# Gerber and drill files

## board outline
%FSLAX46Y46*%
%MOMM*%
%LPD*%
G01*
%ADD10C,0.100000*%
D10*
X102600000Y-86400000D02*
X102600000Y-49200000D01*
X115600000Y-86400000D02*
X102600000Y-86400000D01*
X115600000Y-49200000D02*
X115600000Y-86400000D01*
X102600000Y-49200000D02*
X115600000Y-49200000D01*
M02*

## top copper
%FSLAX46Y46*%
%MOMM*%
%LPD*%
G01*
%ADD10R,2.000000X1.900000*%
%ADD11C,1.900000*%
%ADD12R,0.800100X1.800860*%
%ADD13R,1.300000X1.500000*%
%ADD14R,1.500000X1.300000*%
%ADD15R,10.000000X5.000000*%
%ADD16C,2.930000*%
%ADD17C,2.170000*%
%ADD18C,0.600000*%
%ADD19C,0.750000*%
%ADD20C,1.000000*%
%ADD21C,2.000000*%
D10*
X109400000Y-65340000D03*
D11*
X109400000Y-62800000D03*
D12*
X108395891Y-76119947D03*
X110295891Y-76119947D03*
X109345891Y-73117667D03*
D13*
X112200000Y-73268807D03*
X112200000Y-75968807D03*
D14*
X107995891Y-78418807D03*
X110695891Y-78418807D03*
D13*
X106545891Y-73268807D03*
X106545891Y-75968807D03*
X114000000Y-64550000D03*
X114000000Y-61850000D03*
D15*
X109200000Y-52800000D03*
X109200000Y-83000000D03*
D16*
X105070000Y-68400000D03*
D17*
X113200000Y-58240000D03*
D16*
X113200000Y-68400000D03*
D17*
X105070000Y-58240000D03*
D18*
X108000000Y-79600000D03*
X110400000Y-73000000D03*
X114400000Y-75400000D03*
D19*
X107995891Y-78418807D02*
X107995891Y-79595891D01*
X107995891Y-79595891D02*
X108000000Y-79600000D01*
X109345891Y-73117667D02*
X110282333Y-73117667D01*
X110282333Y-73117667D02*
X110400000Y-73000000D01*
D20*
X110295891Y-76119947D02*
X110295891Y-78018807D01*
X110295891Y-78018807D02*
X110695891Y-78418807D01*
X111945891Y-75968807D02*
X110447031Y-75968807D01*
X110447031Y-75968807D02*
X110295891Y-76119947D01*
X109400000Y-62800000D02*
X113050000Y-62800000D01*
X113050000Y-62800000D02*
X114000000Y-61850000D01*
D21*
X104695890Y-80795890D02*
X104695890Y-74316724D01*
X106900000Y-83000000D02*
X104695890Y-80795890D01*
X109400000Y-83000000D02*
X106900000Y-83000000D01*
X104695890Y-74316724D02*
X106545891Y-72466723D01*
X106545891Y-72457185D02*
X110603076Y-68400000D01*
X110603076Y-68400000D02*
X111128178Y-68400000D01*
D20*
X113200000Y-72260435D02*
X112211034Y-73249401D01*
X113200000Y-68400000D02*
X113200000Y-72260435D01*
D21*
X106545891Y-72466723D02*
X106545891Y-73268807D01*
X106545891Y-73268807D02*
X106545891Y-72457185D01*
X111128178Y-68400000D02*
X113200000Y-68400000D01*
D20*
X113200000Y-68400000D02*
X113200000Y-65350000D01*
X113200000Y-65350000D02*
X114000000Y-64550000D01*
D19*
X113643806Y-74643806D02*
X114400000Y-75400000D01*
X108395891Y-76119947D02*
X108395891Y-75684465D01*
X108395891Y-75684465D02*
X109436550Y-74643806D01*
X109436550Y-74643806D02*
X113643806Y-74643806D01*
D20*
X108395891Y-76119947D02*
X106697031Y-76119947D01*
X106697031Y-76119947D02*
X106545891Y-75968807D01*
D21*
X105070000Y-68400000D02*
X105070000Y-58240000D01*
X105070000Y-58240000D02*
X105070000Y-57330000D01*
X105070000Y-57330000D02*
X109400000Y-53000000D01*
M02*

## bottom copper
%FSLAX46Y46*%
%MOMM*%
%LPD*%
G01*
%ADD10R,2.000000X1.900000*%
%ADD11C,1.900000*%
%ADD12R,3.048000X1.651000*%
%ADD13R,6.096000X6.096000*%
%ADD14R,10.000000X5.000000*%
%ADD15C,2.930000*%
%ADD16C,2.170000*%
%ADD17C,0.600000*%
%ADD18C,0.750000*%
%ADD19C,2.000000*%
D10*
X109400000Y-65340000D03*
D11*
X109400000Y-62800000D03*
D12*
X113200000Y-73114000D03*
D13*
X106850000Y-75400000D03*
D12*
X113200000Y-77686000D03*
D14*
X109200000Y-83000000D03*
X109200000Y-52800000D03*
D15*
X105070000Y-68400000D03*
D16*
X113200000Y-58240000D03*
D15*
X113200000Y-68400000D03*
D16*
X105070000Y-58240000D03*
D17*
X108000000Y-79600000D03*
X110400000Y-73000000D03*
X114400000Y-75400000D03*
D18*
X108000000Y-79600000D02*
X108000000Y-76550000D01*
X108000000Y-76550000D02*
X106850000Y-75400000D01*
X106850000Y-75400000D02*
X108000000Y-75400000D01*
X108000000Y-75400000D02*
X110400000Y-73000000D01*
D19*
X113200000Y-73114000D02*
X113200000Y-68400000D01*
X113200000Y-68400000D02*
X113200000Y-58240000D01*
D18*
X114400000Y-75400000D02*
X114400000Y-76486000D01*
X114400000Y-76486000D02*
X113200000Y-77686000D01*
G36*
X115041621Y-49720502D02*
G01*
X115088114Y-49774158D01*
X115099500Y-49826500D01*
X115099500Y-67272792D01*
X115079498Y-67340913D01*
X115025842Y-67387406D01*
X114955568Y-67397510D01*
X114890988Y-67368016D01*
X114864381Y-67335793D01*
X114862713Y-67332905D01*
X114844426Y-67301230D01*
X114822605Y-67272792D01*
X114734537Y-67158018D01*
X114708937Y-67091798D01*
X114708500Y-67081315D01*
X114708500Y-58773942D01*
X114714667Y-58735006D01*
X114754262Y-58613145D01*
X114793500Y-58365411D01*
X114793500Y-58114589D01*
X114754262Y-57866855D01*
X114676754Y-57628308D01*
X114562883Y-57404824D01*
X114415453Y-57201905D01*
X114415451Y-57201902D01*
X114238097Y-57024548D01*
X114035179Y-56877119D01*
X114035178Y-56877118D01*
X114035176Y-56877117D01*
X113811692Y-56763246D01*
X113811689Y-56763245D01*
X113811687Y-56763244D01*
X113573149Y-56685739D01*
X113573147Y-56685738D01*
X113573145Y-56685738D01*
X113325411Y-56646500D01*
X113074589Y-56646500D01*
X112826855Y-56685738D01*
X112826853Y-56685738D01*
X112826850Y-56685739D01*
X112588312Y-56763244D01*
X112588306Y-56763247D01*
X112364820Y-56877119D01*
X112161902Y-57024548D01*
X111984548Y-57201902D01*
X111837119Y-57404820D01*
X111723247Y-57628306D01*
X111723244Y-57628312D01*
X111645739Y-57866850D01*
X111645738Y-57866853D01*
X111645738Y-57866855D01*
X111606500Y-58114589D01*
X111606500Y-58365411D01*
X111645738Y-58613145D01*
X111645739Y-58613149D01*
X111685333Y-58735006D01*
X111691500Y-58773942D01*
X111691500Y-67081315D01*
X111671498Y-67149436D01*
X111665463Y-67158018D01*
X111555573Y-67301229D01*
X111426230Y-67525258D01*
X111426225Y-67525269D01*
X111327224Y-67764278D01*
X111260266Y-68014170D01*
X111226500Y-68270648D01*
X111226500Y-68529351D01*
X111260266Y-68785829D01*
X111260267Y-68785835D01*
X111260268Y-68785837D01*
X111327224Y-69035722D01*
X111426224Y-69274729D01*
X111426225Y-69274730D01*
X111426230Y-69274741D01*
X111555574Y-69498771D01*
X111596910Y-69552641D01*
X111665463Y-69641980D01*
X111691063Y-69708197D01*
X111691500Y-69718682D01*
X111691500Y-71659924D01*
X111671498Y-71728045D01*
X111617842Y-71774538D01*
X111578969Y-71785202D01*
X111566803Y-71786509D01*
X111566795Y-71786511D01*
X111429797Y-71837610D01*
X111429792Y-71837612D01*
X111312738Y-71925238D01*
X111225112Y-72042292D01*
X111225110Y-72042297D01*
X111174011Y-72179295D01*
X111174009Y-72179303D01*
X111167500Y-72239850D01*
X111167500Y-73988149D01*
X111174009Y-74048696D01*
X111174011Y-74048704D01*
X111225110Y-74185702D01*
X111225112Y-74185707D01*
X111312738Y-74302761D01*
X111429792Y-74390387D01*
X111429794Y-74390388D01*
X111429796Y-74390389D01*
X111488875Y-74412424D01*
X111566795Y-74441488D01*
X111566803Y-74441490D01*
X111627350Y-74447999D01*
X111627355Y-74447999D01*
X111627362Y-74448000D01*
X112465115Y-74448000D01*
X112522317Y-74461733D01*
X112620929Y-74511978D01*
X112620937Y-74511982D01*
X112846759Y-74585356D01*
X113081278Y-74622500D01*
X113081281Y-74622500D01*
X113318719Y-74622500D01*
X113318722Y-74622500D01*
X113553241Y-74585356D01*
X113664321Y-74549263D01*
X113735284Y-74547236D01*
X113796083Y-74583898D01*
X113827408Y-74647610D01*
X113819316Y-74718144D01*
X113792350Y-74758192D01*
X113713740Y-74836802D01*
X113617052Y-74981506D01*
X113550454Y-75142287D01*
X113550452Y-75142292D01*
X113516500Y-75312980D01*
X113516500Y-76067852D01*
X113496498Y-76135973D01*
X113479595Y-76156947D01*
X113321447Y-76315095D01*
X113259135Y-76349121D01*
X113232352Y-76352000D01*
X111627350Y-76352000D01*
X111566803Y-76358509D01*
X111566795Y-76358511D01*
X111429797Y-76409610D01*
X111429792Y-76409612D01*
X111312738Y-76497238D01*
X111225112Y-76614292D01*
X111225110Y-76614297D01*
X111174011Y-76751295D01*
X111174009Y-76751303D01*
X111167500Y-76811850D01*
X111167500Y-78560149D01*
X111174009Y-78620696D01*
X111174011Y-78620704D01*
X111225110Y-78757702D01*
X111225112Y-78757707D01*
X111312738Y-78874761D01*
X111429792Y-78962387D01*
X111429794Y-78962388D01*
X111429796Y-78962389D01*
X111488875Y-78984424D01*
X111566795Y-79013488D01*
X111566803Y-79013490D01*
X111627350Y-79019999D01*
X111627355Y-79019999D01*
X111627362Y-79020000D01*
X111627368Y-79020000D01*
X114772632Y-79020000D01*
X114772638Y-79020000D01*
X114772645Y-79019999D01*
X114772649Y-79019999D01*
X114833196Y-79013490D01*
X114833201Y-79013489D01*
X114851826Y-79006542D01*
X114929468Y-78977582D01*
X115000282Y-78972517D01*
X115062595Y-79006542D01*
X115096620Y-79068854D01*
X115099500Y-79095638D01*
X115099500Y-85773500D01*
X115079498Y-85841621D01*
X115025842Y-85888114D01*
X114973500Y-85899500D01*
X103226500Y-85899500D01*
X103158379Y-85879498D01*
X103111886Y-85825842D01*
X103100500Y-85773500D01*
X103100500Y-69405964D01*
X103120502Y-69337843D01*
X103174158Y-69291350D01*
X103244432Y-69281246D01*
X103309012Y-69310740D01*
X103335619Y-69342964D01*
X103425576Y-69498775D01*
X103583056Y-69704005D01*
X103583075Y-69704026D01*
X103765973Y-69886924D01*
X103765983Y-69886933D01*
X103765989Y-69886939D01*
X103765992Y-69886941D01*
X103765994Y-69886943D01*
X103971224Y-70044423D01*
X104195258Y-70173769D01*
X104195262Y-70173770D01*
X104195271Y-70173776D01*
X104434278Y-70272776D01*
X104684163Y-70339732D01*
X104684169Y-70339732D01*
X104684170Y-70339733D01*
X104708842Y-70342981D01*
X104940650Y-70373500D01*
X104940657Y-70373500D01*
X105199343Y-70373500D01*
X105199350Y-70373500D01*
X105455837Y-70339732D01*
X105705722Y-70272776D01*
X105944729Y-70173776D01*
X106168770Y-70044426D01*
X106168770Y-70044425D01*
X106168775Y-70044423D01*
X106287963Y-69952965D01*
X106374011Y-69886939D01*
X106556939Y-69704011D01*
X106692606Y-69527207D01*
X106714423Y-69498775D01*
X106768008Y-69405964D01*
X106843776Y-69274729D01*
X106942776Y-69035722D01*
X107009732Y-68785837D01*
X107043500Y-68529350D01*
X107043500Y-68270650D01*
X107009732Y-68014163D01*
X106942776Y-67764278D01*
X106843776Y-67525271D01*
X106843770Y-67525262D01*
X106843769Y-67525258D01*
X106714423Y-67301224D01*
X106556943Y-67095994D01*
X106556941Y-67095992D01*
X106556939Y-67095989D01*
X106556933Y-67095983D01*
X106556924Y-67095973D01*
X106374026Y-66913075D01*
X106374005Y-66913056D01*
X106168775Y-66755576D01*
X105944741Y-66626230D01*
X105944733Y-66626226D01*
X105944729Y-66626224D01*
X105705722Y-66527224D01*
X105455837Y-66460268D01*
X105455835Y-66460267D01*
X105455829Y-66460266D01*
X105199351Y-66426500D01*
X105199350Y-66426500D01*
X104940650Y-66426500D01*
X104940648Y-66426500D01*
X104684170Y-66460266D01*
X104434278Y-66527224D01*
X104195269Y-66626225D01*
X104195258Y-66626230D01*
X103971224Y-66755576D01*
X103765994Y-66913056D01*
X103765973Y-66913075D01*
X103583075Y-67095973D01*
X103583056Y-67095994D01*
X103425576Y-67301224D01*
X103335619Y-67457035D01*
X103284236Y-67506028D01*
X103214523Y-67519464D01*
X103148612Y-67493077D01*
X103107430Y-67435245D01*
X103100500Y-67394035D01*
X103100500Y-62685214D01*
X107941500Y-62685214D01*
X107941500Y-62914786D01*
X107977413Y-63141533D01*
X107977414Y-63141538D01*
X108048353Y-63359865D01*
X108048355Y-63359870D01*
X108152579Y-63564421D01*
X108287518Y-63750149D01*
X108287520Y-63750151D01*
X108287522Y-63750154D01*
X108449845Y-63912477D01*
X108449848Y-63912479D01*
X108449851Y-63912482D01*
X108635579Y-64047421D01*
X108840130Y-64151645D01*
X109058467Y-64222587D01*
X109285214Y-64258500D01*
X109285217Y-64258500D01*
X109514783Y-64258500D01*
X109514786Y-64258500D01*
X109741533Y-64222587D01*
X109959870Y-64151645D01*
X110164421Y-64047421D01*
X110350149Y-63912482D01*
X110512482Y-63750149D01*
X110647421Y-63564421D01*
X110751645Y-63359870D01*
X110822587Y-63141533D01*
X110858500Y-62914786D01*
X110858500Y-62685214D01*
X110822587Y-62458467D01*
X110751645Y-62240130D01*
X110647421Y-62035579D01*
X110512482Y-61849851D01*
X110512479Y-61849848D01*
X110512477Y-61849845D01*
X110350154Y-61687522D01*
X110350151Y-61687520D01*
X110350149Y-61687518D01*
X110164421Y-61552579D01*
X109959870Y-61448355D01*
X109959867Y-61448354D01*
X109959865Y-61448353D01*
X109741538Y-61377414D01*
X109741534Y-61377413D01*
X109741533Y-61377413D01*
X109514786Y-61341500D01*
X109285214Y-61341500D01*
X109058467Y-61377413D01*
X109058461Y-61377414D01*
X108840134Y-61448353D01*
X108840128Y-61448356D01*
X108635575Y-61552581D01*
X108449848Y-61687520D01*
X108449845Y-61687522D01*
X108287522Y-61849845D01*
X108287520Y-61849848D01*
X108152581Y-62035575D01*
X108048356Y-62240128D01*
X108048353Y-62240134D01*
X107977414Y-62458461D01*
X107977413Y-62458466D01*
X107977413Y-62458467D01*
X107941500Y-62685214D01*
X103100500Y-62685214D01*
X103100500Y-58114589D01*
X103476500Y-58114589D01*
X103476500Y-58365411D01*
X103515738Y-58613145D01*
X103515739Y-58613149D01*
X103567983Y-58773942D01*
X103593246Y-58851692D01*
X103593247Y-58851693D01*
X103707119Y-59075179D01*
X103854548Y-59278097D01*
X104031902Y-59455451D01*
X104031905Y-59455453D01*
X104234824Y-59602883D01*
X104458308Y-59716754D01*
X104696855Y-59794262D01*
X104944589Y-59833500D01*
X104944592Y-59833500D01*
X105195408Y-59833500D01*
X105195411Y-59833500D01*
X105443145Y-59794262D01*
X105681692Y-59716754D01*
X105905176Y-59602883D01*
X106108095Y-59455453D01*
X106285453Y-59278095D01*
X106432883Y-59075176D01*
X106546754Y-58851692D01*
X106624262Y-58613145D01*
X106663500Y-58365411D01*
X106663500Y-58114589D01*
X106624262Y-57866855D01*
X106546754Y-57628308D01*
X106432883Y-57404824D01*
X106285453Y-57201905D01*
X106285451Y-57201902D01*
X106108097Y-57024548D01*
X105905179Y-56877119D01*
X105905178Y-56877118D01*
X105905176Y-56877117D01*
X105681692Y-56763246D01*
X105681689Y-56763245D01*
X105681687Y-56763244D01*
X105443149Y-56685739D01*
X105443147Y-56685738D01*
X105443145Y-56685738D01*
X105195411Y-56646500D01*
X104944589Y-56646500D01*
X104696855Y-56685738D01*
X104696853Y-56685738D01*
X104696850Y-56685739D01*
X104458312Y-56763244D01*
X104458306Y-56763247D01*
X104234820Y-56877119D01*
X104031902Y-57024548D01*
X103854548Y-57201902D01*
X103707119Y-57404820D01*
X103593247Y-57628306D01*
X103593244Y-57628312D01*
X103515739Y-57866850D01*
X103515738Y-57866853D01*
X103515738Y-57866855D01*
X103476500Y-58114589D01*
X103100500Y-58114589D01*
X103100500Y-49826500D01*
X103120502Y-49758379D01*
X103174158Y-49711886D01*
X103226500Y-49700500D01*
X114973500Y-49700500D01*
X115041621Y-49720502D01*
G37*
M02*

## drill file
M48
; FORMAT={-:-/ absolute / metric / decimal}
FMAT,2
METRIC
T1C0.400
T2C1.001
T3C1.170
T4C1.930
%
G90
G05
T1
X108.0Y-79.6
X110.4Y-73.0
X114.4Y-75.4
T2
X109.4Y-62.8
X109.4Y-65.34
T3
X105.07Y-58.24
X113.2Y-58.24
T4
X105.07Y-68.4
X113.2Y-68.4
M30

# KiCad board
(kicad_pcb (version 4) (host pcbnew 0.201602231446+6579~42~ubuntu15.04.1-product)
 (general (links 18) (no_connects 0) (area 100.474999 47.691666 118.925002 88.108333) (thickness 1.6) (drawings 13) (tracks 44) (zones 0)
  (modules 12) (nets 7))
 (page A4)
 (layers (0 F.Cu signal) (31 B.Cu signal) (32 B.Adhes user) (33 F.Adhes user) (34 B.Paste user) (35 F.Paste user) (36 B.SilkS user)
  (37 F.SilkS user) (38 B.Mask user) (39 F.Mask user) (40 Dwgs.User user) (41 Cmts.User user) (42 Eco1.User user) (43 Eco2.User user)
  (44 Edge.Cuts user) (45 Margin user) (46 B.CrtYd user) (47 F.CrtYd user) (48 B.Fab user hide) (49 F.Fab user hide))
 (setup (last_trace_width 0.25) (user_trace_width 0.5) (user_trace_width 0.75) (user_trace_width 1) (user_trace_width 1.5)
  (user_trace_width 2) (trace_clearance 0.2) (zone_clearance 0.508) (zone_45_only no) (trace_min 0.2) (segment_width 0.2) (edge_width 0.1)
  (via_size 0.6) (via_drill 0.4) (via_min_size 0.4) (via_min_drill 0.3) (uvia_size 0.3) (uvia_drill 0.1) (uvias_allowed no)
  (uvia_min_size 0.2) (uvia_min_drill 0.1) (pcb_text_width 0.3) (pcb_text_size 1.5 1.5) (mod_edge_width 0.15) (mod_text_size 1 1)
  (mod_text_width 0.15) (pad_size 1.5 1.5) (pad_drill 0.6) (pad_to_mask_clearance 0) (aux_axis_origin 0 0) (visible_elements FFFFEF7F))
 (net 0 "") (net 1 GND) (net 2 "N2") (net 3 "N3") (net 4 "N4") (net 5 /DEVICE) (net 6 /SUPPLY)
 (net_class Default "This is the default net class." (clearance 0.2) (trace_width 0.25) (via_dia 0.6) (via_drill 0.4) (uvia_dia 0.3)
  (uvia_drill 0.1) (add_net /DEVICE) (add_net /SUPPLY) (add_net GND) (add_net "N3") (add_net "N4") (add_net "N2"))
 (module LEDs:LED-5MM (layer F.Cu) (at 109.4 65.34 90)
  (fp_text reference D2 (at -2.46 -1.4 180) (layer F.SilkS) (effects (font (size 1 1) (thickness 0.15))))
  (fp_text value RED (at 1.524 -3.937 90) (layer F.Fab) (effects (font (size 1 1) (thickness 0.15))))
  (pad 1 thru_hole rect (at 0 0 180) (size 2 1.9) (drill 1.00076) (layers *.Cu *.Mask F.SilkS) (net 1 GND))
  (pad 2 thru_hole circle (at 2.54 0 90) (size 1.9 1.9) (drill 1.00076) (layers *.Cu *.Mask F.SilkS) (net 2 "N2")))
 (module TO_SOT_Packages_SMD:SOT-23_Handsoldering (layer F.Cu) (at 109.345891 74.618807)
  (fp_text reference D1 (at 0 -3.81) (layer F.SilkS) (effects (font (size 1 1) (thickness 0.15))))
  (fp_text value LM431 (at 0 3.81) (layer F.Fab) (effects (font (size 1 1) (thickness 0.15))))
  (pad 1 smd rect (at -0.95 1.50114) (size 0.8001 1.80086) (layers F.Cu F.Paste F.Mask) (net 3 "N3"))
  (pad 2 smd rect (at 0.95 1.50114) (size 0.8001 1.80086) (layers F.Cu F.Paste F.Mask) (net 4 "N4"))
  (pad 3 smd rect (at 0 -1.50114) (size 0.8001 1.80086) (layers F.Cu F.Paste F.Mask) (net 1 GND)))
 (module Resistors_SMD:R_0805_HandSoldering (layer F.Cu) (at 112.2 74.618807 270)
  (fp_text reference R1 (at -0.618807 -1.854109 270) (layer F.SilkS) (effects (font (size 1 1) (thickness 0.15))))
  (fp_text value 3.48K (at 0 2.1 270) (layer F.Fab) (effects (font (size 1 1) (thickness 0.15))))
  (pad 1 smd rect (at -1.35 0 270) (size 1.5 1.3) (layers F.Cu F.Paste F.Mask) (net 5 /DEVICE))
  (pad 2 smd rect (at 1.35 0 270) (size 1.5 1.3) (layers F.Cu F.Paste F.Mask) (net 4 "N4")))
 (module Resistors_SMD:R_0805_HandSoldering (layer F.Cu) (at 109.345891 78.418807)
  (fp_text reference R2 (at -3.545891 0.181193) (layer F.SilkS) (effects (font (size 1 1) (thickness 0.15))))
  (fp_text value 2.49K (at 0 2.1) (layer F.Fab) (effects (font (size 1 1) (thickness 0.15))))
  (pad 1 smd rect (at -1.35 0) (size 1.5 1.3) (layers F.Cu F.Paste F.Mask) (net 1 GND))
  (pad 2 smd rect (at 1.35 0) (size 1.5 1.3) (layers F.Cu F.Paste F.Mask) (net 4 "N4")))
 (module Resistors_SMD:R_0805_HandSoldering (layer F.Cu) (at 106.545891 74.618807 270)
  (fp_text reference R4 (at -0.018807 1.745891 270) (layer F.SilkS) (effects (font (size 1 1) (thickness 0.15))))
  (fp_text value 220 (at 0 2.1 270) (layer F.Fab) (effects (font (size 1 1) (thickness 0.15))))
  (pad 1 smd rect (at -1.35 0 270) (size 1.5 1.3) (layers F.Cu F.Paste F.Mask) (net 5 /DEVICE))
  (pad 2 smd rect (at 1.35 0 270) (size 1.5 1.3) (layers F.Cu F.Paste F.Mask) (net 3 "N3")))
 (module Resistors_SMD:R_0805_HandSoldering (layer F.Cu) (at 114 63.2 90)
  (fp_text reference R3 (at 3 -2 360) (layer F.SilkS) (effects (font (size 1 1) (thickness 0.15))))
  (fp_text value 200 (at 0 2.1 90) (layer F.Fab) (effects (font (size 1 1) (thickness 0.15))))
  (pad 1 smd rect (at -1.35 0 90) (size 1.5 1.3) (layers F.Cu F.Paste F.Mask) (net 5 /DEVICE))
  (pad 2 smd rect (at 1.35 0 90) (size 1.5 1.3) (layers F.Cu F.Paste F.Mask) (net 2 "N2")))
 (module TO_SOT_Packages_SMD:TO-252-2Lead (layer B.Cu) (at 113.2 75.4 270)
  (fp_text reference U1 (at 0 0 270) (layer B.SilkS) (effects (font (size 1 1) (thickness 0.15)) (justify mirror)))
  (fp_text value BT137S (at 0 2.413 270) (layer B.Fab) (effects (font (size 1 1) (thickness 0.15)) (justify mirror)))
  (pad 1 smd rect (at -2.286 0 270) (size 1.651 3.048) (layers B.Cu B.Paste B.Mask) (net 5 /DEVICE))
  (pad 2 smd rect (at 0 6.35 270) (size 6.096 6.096) (layers B.Cu B.Paste B.Mask) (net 1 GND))
  (pad 3 smd rect (at 2.286 0 270) (size 1.651 3.048) (layers B.Cu B.Paste B.Mask) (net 3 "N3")))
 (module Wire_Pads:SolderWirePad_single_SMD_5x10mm (layer F.Cu) (at 109.2 52.8 90)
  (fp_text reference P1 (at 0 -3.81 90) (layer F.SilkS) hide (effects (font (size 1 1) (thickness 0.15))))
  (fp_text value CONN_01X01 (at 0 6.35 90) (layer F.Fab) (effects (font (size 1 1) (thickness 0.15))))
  (pad 1 smd rect (at 0 0 90) (size 5 10) (layers F.Cu F.Paste F.Mask) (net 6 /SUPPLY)))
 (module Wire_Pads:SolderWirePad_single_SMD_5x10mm (layer F.Cu) (at 109.2 83 90)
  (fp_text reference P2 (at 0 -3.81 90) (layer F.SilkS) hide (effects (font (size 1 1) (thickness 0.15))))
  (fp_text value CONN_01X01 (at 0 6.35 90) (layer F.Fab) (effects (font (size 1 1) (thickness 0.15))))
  (pad 1 smd rect (at 0 0 90) (size 5 10) (layers F.Cu F.Paste F.Mask) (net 5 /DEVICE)))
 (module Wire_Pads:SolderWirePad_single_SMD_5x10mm (layer B.Cu) (at 109.2 83 90)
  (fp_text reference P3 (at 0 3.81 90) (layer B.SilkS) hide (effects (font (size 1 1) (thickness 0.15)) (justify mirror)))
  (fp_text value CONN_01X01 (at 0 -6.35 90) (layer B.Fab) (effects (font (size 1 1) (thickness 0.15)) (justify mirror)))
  (pad 1 smd rect (at 0 0 90) (size 5 10) (layers B.Cu B.Paste B.Mask) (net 1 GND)))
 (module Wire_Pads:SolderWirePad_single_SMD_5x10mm (layer B.Cu) (at 109.2 52.8 90)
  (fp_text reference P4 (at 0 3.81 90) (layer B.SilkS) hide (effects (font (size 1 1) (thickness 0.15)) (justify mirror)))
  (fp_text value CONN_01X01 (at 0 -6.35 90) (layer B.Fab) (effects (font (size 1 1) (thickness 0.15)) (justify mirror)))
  (pad 1 smd rect (at 0 0 90) (size 5 10) (layers B.Cu B.Paste B.Mask) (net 1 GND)))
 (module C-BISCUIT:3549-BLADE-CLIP (layer B.Cu) (at 109.135 63.32)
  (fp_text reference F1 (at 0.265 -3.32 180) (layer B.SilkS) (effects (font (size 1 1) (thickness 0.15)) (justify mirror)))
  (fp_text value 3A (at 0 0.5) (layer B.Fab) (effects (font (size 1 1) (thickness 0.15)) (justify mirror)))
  (pad 1 thru_hole circle (at -4.065 5.08) (size 2.93 2.93) (drill 1.93) (layers *.Cu *.Mask B.SilkS) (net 6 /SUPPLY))
  (pad 2 thru_hole circle (at 4.065 -5.08) (size 2.17 2.17) (drill 1.17) (layers *.Cu *.Mask B.SilkS) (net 5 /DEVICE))
  (pad 2 thru_hole circle (at 4.065 5.08) (size 2.93 2.93) (drill 1.93) (layers *.Cu *.Mask B.SilkS) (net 5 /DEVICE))
  (pad 1 thru_hole circle (at -4.065 -5.08) (size 2.17 2.17) (drill 1.17) (layers *.Cu *.Mask B.SilkS) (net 6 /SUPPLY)))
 (gr_line (start 102.6 86.4) (end 102.6 49.2) (layer Edge.Cuts) (width 0.1))
 (gr_line (start 115.6 86.4) (end 102.6 86.4) (layer Edge.Cuts) (width 0.1))
 (gr_line (start 115.6 49.2) (end 115.6 86.4) (layer Edge.Cuts) (width 0.1))
 (gr_line (start 102.6 49.2) (end 115.6 49.2) (layer Edge.Cuts) (width 0.1))
 (segment (start 100.8 48.8) (end 118.6 48.8) (width 0.25) (layer Dwgs.User) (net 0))
 (segment (start 108 79.6) (end 108 76.55) (width 0.75) (layer B.Cu) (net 1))
 (segment (start 108 76.55) (end 106.85 75.4) (width 0.75) (layer B.Cu) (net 1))
 (segment (start 107.995891 78.418807) (end 107.995891 79.595891) (width 0.75) (layer F.Cu) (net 1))
 (segment (start 107.995891 79.595891) (end 108 79.6) (width 0.75) (layer F.Cu) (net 1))
 (via (at 108 79.6) (size 0.6) (drill 0.4) (layers F.Cu B.Cu) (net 1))
 (segment (start 106.85 75.4) (end 108 75.4) (width 0.75) (layer B.Cu) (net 1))
 (segment (start 108 75.4) (end 110.4 73) (width 0.75) (layer B.Cu) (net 1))
 (segment (start 109.345891 73.117667) (end 110.282333 73.117667) (width 0.75) (layer F.Cu) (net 1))
 (via (at 110.4 73) (size 0.6) (drill 0.4) (layers F.Cu B.Cu) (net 1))
 (segment (start 110.282333 73.117667) (end 110.4 73) (width 0.75) (layer F.Cu) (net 1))
 (segment (start 110.295891 76.119947) (end 110.295891 78.018807) (width 1) (layer F.Cu) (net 4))
 (segment (start 110.295891 78.018807) (end 110.695891 78.418807) (width 1) (layer F.Cu) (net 4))
 (segment (start 111.945891 75.968807) (end 110.447031 75.968807) (width 1) (layer F.Cu) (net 4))
 (segment (start 110.447031 75.968807) (end 110.295891 76.119947) (width 1) (layer F.Cu) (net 4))
 (segment (start 109.4 62.8) (end 113.05 62.8) (width 1) (layer F.Cu) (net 2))
 (segment (start 113.05 62.8) (end 114 61.85) (width 1) (layer F.Cu) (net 2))
 (segment (start 104.69589 80.79589) (end 104.69589 74.316724) (width 2) (layer F.Cu) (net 5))
 (segment (start 106.9 83) (end 104.69589 80.79589) (width 2) (layer F.Cu) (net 5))
 (segment (start 109.4 83) (end 106.9 83) (width 2) (layer F.Cu) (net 5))
 (segment (start 104.69589 74.316724) (end 106.545891 72.466723) (width 2) (layer F.Cu) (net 5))
 (segment (start 106.545891 72.457185) (end 110.603076 68.4) (width 2) (layer F.Cu) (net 5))
 (segment (start 110.603076 68.4) (end 111.128178 68.4) (width 2) (layer F.Cu) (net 5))
 (segment (start 113.2 72.260435) (end 112.211034 73.249401) (width 1) (layer F.Cu) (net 5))
 (segment (start 113.2 68.4) (end 113.2 72.260435) (width 1) (layer F.Cu) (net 5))
 (segment (start 106.545891 72.466723) (end 106.545891 73.268807) (width 2) (layer F.Cu) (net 5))
 (segment (start 106.545891 73.268807) (end 106.545891 72.457185) (width 2) (layer F.Cu) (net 5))
 (segment (start 111.128178 68.4) (end 113.2 68.4) (width 2) (layer F.Cu) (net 5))
 (segment (start 113.2 73.114) (end 113.2 68.4) (width 2) (layer B.Cu) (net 5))
 (segment (start 113.2 68.4) (end 113.2 65.35) (width 1) (layer F.Cu) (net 5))
 (segment (start 113.2 65.35) (end 114 64.55) (width 1) (layer F.Cu) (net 5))
 (segment (start 113.2 68.4) (end 113.2 58.24) (width 2) (layer B.Cu) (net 5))
 (segment (start 113.643806 74.643806) (end 114.4 75.4) (width 0.75) (layer F.Cu) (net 3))
 (segment (start 108.395891 76.119947) (end 108.395891 75.684465) (width 0.75) (layer F.Cu) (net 3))
 (segment (start 108.395891 75.684465) (end 109.43655 74.643806) (width 0.75) (layer F.Cu) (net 3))
 (segment (start 109.43655 74.643806) (end 113.643806 74.643806) (width 0.75) (layer F.Cu) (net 3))
 (segment (start 108.395891 76.119947) (end 106.697031 76.119947) (width 1) (layer F.Cu) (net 3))
 (segment (start 106.697031 76.119947) (end 106.545891 75.968807) (width 1) (layer F.Cu) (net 3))
 (segment (start 114.4 75.4) (end 114.4 76.486) (width 0.75) (layer B.Cu) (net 3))
 (via (at 114.4 75.4) (size 0.6) (drill 0.4) (layers F.Cu B.Cu) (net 3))
 (segment (start 114.4 76.486) (end 113.2 77.686) (width 0.75) (layer B.Cu) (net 3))
 (segment (start 105.07 68.4) (end 105.07 58.24) (width 2) (layer F.Cu) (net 6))
 (segment (start 105.07 58.24) (end 105.07 57.33) (width 2) (layer F.Cu) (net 6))
 (segment (start 105.07 57.33) (end 109.4 53) (width 2) (layer F.Cu) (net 6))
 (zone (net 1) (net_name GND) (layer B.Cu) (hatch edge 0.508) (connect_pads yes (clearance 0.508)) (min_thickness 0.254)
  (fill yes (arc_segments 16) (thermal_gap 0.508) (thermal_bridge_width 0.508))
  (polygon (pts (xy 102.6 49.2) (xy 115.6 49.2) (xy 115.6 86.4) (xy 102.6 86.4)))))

